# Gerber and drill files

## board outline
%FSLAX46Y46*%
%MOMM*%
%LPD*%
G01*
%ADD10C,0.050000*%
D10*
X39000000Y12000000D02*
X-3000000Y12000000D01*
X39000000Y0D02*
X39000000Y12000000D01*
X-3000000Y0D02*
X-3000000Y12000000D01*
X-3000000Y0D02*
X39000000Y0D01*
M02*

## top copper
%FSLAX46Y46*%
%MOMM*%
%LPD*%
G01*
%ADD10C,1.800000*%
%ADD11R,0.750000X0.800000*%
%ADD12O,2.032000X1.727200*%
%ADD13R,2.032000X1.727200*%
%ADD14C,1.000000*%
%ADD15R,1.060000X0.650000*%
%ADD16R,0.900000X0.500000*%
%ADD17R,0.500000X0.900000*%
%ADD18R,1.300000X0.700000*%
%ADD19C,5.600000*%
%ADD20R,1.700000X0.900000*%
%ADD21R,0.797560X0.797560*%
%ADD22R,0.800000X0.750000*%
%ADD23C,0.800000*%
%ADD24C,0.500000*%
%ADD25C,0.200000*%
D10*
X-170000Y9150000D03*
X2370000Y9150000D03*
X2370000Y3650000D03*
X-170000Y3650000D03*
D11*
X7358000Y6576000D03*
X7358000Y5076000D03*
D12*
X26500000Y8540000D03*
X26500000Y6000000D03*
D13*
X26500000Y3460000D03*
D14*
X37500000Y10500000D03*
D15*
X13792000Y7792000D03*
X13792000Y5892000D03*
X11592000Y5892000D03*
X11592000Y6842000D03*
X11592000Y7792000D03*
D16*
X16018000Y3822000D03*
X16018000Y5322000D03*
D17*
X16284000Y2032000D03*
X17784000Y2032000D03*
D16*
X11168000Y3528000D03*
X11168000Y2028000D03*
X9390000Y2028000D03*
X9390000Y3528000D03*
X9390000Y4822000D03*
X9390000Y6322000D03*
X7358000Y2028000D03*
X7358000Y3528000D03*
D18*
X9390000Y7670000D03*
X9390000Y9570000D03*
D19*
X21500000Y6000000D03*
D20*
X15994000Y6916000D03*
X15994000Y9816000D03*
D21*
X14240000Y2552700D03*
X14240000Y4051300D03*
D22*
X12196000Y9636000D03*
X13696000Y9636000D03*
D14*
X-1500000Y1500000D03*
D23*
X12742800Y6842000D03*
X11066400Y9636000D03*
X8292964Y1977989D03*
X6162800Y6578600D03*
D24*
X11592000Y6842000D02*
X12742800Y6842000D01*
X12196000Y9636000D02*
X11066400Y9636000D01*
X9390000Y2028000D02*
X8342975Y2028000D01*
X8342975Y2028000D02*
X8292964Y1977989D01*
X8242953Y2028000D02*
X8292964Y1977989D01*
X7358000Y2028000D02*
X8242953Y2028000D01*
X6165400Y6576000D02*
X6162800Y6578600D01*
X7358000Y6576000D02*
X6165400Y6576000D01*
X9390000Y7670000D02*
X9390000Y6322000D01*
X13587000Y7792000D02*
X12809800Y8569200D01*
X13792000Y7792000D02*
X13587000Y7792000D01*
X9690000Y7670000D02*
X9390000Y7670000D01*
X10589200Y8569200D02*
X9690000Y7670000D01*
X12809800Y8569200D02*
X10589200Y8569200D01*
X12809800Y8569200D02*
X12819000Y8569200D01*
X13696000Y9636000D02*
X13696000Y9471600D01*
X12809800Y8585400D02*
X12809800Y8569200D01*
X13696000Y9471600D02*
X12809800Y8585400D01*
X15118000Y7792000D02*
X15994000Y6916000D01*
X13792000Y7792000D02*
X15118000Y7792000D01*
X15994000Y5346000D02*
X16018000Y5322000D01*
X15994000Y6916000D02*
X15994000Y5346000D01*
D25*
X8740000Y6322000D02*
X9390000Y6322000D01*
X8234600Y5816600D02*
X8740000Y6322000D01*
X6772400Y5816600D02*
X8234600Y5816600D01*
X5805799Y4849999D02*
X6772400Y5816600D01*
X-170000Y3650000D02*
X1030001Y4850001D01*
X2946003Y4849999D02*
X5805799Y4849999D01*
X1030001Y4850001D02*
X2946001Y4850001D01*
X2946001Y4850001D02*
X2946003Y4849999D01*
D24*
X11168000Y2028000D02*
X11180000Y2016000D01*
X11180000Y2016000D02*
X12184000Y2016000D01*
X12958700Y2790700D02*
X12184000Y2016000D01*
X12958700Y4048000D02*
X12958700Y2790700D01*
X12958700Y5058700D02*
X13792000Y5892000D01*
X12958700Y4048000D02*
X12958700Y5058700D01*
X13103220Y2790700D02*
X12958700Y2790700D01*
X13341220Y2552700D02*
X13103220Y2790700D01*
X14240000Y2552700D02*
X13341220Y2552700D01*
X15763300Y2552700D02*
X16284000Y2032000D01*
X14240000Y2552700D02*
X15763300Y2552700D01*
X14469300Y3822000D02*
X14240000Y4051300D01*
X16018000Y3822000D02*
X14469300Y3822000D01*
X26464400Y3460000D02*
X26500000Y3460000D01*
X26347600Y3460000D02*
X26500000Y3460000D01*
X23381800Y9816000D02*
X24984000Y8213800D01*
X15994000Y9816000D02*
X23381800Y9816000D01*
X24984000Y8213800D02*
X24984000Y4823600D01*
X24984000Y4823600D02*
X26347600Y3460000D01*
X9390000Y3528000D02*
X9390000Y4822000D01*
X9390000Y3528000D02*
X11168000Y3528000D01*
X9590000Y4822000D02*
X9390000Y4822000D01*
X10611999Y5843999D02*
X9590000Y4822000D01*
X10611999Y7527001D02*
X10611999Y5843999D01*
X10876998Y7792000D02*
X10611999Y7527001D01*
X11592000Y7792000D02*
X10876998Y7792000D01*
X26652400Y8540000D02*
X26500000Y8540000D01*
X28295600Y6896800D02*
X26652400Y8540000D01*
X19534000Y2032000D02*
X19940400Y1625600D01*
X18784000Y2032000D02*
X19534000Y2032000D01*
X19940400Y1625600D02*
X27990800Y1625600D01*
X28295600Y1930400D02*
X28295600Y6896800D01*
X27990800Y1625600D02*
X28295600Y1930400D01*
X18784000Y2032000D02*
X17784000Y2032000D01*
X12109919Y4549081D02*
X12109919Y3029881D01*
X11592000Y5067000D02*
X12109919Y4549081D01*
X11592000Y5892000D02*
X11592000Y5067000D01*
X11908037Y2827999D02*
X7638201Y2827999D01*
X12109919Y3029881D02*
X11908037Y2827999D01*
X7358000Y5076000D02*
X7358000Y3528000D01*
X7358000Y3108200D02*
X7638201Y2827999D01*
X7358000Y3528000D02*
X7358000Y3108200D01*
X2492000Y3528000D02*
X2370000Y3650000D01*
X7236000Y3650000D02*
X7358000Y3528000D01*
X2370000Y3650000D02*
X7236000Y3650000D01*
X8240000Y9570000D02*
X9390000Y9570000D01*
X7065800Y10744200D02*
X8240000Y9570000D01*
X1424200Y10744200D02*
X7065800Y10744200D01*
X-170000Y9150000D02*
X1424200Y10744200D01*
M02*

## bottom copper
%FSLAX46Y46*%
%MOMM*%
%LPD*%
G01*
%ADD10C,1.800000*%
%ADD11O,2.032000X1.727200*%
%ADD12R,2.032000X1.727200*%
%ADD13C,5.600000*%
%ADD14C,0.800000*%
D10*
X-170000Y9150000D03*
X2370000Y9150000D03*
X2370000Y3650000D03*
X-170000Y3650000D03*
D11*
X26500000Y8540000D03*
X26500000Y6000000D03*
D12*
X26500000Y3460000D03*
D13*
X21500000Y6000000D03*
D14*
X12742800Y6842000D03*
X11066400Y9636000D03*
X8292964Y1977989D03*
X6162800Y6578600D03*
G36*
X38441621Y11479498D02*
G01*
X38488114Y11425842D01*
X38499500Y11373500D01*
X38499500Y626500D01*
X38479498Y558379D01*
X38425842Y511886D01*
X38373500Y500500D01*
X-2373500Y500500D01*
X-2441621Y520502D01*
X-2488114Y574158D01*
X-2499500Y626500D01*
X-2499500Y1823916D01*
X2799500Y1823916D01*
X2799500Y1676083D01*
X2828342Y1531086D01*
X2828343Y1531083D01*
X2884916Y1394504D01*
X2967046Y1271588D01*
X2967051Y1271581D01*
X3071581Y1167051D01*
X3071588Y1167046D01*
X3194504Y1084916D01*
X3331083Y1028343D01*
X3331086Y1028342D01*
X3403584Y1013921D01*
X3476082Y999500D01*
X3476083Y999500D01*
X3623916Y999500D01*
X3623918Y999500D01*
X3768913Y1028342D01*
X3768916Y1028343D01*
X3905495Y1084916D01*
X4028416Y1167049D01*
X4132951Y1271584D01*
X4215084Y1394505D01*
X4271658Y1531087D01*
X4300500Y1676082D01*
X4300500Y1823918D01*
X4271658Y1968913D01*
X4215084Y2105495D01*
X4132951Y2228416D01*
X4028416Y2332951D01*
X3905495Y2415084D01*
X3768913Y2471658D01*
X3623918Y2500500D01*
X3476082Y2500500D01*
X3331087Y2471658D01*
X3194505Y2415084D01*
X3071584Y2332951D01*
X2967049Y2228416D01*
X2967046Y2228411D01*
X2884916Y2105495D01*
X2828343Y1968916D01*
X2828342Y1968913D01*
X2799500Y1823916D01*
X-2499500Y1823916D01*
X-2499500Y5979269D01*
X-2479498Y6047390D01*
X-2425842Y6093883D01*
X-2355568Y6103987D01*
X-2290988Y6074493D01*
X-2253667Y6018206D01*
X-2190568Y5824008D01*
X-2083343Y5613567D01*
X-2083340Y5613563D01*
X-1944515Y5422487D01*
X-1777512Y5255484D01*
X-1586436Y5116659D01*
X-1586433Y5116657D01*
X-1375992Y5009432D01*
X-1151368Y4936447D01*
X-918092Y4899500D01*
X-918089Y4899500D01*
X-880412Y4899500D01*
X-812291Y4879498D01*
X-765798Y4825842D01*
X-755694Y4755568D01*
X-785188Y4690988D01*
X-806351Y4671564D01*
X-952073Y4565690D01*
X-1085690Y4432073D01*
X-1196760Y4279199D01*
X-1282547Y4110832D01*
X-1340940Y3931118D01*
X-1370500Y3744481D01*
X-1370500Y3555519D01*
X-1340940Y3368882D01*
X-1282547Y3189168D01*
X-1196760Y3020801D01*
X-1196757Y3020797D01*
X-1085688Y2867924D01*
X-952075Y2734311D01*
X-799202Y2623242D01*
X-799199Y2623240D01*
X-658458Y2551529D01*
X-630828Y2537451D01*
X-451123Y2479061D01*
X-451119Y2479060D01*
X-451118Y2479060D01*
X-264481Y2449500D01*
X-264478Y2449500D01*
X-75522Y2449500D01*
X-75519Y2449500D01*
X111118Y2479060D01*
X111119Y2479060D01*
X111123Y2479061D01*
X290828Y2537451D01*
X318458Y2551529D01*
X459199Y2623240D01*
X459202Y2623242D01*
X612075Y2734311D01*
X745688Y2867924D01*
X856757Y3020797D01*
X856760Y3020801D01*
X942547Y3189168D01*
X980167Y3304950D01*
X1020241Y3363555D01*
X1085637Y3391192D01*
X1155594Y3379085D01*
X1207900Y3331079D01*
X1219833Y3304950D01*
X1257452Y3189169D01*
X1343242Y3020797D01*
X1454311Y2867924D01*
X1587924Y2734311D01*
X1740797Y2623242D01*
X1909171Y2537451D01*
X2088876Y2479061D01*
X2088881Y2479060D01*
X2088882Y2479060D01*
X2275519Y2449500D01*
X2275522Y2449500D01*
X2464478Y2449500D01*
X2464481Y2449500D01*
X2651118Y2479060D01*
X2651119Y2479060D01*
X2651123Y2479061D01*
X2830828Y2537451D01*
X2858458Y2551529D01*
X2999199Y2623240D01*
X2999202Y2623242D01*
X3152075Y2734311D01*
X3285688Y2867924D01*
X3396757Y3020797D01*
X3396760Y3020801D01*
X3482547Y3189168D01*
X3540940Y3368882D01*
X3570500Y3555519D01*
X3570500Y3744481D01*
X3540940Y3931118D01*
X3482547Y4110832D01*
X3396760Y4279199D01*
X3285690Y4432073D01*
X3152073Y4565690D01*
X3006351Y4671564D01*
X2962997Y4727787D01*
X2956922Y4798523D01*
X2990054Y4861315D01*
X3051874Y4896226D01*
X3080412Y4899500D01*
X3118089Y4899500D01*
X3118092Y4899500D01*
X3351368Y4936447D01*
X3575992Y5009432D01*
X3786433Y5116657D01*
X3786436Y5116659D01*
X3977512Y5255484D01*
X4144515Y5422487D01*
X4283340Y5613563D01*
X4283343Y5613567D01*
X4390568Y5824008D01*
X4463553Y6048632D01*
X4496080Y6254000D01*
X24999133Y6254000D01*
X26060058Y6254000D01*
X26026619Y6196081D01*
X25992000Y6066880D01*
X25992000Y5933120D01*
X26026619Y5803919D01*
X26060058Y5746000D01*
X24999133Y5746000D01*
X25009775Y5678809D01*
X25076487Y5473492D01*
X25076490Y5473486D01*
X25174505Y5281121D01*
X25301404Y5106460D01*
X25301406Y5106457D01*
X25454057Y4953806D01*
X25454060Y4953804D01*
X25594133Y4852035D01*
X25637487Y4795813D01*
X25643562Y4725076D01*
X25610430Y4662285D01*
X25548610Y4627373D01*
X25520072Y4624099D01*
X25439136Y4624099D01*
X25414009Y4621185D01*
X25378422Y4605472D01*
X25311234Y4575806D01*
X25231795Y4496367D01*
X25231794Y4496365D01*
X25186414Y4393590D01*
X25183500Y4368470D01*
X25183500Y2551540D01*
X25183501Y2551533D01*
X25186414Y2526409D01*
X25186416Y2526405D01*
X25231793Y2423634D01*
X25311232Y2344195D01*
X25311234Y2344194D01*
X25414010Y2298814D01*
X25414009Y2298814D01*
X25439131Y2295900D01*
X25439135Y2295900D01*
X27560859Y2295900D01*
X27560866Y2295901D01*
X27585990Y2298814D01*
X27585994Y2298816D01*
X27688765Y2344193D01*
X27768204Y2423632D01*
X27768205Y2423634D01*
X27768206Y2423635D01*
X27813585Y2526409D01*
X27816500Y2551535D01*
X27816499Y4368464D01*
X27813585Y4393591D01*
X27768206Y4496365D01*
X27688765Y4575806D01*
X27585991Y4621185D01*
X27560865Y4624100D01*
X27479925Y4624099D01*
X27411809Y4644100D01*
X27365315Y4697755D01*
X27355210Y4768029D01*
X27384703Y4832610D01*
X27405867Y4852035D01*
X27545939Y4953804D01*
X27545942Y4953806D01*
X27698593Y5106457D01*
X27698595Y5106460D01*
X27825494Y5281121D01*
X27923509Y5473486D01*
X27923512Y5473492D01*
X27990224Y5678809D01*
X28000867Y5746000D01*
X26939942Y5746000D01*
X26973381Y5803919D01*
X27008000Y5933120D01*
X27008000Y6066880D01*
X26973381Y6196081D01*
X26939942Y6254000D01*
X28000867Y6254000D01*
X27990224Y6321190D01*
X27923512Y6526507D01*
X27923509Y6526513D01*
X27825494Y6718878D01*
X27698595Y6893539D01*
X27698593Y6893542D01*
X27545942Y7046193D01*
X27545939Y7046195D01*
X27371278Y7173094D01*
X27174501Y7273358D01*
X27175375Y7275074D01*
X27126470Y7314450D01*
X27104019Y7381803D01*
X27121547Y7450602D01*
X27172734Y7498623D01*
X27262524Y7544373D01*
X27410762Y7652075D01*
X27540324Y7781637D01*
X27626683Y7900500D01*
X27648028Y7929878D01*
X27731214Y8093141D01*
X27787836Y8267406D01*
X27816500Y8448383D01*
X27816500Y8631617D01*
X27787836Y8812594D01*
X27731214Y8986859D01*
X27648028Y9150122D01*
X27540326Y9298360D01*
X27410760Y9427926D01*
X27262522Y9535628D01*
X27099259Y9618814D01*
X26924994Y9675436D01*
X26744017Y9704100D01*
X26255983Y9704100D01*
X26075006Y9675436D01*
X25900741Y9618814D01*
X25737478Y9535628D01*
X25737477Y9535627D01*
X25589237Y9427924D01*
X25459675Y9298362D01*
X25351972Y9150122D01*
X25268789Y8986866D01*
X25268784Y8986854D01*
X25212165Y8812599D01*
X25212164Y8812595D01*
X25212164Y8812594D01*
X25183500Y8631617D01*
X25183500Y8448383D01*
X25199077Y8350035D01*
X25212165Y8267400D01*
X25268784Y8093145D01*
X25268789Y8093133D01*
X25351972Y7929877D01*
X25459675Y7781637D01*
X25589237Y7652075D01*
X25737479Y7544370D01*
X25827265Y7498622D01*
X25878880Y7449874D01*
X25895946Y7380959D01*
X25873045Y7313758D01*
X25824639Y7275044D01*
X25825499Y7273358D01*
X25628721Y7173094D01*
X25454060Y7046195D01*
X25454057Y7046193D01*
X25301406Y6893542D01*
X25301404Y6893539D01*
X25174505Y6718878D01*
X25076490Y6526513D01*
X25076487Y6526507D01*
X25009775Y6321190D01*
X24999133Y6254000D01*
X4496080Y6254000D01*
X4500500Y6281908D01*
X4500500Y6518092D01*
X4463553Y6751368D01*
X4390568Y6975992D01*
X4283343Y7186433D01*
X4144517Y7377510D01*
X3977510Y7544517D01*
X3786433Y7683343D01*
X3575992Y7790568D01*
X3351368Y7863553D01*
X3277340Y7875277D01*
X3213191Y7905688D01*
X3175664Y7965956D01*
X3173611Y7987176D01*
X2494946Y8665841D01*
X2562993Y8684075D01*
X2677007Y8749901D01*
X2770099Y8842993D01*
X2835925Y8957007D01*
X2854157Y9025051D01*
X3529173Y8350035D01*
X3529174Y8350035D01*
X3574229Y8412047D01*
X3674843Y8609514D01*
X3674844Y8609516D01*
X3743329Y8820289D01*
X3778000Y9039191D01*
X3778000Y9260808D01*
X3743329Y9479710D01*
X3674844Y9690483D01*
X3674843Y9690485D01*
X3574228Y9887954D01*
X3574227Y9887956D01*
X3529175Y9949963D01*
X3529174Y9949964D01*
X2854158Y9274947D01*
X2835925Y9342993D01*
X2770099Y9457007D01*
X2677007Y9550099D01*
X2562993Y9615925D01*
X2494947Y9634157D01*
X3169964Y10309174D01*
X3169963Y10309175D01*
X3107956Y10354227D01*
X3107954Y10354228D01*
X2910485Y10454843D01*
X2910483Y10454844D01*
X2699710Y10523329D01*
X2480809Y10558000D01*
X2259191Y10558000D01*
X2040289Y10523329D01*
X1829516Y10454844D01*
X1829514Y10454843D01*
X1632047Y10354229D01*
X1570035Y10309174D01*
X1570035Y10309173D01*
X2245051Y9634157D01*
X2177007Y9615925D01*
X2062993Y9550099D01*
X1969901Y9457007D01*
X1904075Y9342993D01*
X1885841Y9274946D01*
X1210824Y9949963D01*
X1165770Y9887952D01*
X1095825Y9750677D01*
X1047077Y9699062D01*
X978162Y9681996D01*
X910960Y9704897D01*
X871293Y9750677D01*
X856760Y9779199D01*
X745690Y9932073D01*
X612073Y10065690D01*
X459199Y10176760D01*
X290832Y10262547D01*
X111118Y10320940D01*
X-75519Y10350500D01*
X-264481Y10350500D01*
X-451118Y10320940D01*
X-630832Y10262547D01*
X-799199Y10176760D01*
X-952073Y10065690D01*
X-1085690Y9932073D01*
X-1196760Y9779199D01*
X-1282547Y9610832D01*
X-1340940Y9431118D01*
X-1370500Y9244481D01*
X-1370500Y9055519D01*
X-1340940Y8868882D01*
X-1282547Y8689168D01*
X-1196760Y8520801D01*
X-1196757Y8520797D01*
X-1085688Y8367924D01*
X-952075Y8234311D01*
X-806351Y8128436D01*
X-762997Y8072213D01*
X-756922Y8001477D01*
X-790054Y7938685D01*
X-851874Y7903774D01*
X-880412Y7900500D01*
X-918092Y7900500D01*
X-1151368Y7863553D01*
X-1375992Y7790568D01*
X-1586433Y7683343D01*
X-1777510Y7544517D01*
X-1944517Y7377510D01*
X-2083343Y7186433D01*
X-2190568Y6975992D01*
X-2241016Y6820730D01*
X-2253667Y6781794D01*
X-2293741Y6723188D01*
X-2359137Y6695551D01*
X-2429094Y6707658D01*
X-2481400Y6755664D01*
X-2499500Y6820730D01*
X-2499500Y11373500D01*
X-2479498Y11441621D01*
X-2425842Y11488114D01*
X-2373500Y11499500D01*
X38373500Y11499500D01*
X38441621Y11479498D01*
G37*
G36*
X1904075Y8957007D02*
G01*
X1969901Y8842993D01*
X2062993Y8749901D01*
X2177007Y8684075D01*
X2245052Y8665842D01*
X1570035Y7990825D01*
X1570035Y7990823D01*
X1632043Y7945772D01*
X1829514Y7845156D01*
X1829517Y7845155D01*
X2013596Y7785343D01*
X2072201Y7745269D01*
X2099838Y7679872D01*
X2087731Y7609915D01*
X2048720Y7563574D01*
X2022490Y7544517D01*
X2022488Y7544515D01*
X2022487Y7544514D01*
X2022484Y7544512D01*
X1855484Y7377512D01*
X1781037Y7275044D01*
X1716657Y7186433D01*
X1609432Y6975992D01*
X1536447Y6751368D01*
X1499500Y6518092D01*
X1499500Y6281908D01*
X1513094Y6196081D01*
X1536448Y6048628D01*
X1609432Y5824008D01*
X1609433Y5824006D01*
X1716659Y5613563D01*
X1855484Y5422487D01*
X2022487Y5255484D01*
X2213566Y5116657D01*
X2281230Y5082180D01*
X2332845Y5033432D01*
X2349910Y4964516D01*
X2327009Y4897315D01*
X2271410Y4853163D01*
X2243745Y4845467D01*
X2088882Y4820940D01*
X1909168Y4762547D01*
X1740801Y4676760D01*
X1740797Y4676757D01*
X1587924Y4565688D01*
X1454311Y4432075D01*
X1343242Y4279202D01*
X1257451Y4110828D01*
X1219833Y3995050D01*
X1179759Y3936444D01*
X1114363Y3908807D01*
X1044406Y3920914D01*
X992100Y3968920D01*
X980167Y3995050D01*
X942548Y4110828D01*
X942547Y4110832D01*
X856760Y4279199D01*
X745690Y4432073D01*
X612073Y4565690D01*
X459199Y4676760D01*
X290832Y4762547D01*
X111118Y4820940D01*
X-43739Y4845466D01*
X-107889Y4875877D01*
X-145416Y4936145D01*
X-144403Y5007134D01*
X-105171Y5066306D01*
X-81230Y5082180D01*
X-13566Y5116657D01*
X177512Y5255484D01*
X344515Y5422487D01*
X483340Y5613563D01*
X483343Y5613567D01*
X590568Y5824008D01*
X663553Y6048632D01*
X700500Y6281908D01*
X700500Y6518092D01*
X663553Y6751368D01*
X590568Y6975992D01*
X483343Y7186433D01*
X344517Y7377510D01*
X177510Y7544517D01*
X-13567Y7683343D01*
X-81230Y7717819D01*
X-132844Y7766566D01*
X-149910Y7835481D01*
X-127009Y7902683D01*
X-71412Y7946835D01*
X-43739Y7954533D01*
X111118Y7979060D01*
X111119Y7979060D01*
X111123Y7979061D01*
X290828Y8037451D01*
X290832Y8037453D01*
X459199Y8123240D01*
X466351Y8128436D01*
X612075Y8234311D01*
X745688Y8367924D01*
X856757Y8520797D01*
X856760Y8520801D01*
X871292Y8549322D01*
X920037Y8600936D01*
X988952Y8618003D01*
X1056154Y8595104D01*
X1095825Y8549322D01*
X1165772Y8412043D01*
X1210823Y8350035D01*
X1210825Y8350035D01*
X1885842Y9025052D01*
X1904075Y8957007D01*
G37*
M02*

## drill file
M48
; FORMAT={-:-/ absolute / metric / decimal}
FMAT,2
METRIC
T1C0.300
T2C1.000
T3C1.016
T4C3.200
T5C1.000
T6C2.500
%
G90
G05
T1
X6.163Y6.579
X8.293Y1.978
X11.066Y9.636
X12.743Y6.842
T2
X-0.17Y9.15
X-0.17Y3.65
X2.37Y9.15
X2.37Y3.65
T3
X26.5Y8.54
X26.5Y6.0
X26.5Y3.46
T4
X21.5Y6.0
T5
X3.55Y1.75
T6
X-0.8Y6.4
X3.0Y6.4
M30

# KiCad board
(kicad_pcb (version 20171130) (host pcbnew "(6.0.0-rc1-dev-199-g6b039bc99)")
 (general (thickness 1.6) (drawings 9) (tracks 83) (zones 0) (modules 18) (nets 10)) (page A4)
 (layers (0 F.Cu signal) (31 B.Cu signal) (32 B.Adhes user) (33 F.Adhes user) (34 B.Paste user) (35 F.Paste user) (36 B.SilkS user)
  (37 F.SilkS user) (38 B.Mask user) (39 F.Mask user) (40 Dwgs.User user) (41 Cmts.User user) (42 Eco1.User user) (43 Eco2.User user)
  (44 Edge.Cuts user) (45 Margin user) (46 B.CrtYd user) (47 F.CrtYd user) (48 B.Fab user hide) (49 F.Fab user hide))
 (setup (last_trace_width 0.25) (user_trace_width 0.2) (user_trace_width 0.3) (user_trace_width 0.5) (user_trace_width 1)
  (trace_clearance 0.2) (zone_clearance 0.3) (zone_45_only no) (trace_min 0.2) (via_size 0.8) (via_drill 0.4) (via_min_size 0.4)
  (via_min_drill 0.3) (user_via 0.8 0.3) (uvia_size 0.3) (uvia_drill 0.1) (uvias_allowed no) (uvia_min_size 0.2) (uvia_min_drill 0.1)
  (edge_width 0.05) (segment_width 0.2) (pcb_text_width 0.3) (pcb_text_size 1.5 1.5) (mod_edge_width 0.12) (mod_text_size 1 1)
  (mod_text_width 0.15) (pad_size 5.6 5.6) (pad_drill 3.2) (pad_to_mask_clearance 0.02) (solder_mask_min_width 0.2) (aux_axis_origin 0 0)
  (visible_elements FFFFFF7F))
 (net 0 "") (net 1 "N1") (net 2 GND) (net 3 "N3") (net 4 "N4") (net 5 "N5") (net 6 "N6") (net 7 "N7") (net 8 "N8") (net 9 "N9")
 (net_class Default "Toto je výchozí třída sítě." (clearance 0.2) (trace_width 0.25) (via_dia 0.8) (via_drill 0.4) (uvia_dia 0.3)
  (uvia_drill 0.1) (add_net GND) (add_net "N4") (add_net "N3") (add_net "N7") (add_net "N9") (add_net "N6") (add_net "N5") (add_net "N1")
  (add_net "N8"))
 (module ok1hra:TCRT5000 (layer F.Cu) (at 1.1 -6.4 90)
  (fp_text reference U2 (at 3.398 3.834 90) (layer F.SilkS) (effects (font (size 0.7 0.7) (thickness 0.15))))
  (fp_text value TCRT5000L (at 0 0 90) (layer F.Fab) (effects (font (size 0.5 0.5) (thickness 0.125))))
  (pad "" np_thru_hole circle (at -4.65 2.45 90) (size 1 1) (drill 1) (layers *.Cu *.Mask))
  (pad "" np_thru_hole circle (at 0 1.9 90) (size 2.5 2.5) (drill 2.5) (layers *.Cu *.Mask))
  (pad "" np_thru_hole circle (at 0 -1.9 90) (size 2.5 2.5) (drill 2.5) (layers *.Cu *.Mask))
  (pad 4 thru_hole circle (at 2.75 -1.27 90) (size 1.8 1.8) (drill 1) (layers *.Cu *.Mask) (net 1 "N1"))
  (pad 3 thru_hole circle (at 2.75 1.27 90) (size 1.8 1.8) (drill 1) (layers *.Cu *.Mask) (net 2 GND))
  (pad 2 thru_hole circle (at -2.75 1.27 90) (size 1.8 1.8) (drill 1) (layers *.Cu *.Mask) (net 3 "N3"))
  (pad 1 thru_hole circle (at -2.75 -1.27 90) (size 1.8 1.8) (drill 1) (layers *.Cu *.Mask) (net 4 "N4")))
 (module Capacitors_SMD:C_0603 (layer F.Cu) (at 7.358 -5.826 90)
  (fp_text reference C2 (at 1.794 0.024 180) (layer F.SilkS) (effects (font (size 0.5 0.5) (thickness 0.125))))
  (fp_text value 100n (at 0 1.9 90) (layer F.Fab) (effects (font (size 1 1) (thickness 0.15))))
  (pad 2 smd rect (at 0.75 0 90) (size 0.8 0.75) (layers F.Cu F.Paste F.Mask) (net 2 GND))
  (pad 1 smd rect (at -0.75 0 90) (size 0.8 0.75) (layers F.Cu F.Paste F.Mask) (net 3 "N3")))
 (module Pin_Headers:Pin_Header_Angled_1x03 (layer B.Cu) (at 26.5 -3.46)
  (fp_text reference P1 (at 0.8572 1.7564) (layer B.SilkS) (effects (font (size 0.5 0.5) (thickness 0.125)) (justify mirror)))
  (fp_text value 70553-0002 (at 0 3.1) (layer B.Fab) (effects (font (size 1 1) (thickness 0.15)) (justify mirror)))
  (pad 3 thru_hole oval (at 0 -5.08) (size 2.032 1.7272) (drill 1.016) (layers *.Cu *.Mask) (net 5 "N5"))
  (pad 2 thru_hole oval (at 0 -2.54) (size 2.032 1.7272) (drill 1.016) (layers *.Cu *.Mask) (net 2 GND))
  (pad 1 thru_hole rect (at 0 0) (size 2.032 1.7272) (drill 1.016) (layers *.Cu *.Mask) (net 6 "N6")))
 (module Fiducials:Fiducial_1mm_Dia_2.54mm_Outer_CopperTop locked (layer F.Cu) (at 37.5 -10.5)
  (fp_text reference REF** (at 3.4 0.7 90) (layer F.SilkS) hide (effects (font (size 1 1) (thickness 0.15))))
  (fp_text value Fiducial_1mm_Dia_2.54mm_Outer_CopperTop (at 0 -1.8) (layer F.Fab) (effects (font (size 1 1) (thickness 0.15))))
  (pad ~ smd circle (at 0 0) (size 1 1) (layers F.Cu F.Mask) (solder_mask_margin 0.77) (clearance 0.77)))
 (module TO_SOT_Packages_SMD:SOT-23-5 (layer F.Cu) (at 12.692 -6.842)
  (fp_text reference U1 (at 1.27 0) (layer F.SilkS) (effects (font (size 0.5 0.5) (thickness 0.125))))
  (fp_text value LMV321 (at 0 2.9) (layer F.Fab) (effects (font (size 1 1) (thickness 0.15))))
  (pad 5 smd rect (at 1.1 -0.95) (size 1.06 0.65) (layers F.Cu F.Paste F.Mask) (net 4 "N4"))
  (pad 4 smd rect (at 1.1 0.95) (size 1.06 0.65) (layers F.Cu F.Paste F.Mask) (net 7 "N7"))
  (pad 3 smd rect (at -1.1 0.95) (size 1.06 0.65) (layers F.Cu F.Paste F.Mask) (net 3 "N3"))
  (pad 2 smd rect (at -1.1 0) (size 1.06 0.65) (layers F.Cu F.Paste F.Mask) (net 2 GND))
  (pad 1 smd rect (at -1.1 -0.95) (size 1.06 0.65) (layers F.Cu F.Paste F.Mask) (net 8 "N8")))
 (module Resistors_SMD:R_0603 (layer F.Cu) (at 16.018 -4.572 270)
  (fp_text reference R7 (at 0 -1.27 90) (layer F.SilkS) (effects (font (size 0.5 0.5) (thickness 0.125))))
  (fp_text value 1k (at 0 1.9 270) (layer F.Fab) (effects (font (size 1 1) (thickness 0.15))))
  (pad 2 smd rect (at 0.75 0 270) (size 0.5 0.9) (layers F.Cu F.Paste F.Mask) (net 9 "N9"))
  (pad 1 smd rect (at -0.75 0 270) (size 0.5 0.9) (layers F.Cu F.Paste F.Mask) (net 4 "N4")))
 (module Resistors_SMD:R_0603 (layer F.Cu) (at 17.034 -2.032 180)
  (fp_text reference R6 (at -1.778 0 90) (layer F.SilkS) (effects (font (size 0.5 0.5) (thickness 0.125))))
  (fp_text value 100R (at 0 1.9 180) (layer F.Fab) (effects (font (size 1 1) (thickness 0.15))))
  (pad 2 smd rect (at 0.75 0 180) (size 0.5 0.9) (layers F.Cu F.Paste F.Mask) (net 7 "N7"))
  (pad 1 smd rect (at -0.75 0 180) (size 0.5 0.9) (layers F.Cu F.Paste F.Mask) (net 5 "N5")))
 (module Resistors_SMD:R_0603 (layer F.Cu) (at 11.168 -2.778 90)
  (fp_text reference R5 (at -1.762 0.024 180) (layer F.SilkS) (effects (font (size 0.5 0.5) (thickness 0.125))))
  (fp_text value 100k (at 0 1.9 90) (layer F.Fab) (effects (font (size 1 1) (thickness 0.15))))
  (pad 2 smd rect (at 0.75 0 90) (size 0.5 0.9) (layers F.Cu F.Paste F.Mask) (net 8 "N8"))
  (pad 1 smd rect (at -0.75 0 90) (size 0.5 0.9) (layers F.Cu F.Paste F.Mask) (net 7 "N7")))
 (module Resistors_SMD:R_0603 (layer F.Cu) (at 9.39 -2.778 270)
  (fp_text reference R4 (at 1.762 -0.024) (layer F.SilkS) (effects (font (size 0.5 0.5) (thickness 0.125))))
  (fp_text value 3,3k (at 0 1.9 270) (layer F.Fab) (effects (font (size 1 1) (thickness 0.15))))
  (pad 2 smd rect (at 0.75 0 270) (size 0.5 0.9) (layers F.Cu F.Paste F.Mask) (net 2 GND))
  (pad 1 smd rect (at -0.75 0 270) (size 0.5 0.9) (layers F.Cu F.Paste F.Mask) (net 8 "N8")))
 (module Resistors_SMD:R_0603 (layer F.Cu) (at 9.39 -5.572 270)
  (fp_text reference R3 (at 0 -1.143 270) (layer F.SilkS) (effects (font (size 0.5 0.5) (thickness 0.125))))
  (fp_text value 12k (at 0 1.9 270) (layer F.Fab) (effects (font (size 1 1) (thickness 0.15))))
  (pad 2 smd rect (at 0.75 0 270) (size 0.5 0.9) (layers F.Cu F.Paste F.Mask) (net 8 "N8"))
  (pad 1 smd rect (at -0.75 0 270) (size 0.5 0.9) (layers F.Cu F.Paste F.Mask) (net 4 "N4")))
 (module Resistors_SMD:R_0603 (layer F.Cu) (at 7.358 -2.778 270)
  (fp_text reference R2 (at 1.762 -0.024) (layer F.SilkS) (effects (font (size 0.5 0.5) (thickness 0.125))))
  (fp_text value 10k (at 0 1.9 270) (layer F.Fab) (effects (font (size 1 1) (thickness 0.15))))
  (pad 2 smd rect (at 0.75 0 270) (size 0.5 0.9) (layers F.Cu F.Paste F.Mask) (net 2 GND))
  (pad 1 smd rect (at -0.75 0 270) (size 0.5 0.9) (layers F.Cu F.Paste F.Mask) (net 3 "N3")))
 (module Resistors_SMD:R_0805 (layer F.Cu) (at 9.39 -8.62 270)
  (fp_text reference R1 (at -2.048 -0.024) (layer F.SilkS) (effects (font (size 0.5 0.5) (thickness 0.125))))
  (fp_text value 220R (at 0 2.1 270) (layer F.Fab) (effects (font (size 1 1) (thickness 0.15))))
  (pad 2 smd rect (at 0.95 0 270) (size 0.7 1.3) (layers F.Cu F.Paste F.Mask) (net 4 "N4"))
  (pad 1 smd rect (at -0.95 0 270) (size 0.7 1.3) (layers F.Cu F.Paste F.Mask) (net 1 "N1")))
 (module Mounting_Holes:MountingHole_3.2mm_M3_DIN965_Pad (layer F.Cu) (at 21.5 -6)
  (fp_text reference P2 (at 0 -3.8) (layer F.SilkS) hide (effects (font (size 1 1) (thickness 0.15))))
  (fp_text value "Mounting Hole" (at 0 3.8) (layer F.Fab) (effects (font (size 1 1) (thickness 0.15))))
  (pad 1 thru_hole circle (at 0 0) (size 5.6 5.6) (drill 3.2) (layers *.Cu *.Mask) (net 2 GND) (zone_connect 2)))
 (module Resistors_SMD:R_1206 (layer F.Cu) (at 15.994 -8.366 270)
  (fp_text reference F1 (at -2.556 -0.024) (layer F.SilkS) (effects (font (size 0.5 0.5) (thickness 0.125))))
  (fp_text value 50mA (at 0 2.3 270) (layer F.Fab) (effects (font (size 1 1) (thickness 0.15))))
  (pad 2 smd rect (at 1.45 0 270) (size 0.9 1.7) (layers F.Cu F.Paste F.Mask) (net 4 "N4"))
  (pad 1 smd rect (at -1.45 0 270) (size 0.9 1.7) (layers F.Cu F.Paste F.Mask) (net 6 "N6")))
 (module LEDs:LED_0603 (layer F.Cu) (at 14.24 -3.302 90)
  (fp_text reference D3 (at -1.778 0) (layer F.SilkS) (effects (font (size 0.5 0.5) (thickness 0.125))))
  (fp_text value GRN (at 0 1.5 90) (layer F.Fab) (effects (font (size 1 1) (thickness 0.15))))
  (pad 1 smd rect (at -0.7493 0 270) (size 0.79756 0.79756) (layers F.Cu F.Paste F.Mask) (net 7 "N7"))
  (pad 2 smd rect (at 0.7493 0 270) (size 0.79756 0.79756) (layers F.Cu F.Paste F.Mask) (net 9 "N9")))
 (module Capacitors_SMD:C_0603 (layer F.Cu) (at 12.946 -9.636 180)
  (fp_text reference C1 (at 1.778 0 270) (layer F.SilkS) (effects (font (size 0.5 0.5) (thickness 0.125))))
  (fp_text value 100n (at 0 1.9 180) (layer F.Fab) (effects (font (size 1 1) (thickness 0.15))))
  (pad 2 smd rect (at 0.75 0 180) (size 0.8 0.75) (layers F.Cu F.Paste F.Mask) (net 2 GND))
  (pad 1 smd rect (at -0.75 0 180) (size 0.8 0.75) (layers F.Cu F.Paste F.Mask) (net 4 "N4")))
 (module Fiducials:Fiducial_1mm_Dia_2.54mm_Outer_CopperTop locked (layer F.Cu) (at -1.5 -1.5)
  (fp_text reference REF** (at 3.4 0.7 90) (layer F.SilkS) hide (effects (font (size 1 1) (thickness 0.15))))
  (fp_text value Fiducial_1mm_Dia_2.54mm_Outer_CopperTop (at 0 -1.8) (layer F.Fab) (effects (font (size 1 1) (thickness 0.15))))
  (pad ~ smd circle (at 0 0) (size 1 1) (layers F.Cu F.Mask) (solder_mask_margin 0.77) (clearance 0.77)))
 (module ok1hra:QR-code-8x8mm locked (layer B.Cu) (at 11 -6 180)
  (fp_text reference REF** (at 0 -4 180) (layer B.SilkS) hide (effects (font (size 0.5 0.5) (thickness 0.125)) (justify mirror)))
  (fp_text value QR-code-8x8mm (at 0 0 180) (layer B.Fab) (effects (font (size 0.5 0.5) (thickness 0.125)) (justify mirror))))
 (gr_line (start 39 -12) (end -3 -12) (layer Edge.Cuts) (width 0.05))
 (gr_line (start 39 0) (end 39 -12) (layer Edge.Cuts) (width 0.05))
 (gr_line (start -3 0) (end -3 -12) (layer Edge.Cuts) (width 0.05))
 (gr_line (start -3 0) (end 39 0) (layer Edge.Cuts) (width 0.05))
 (via (at 12.7428 -6.842) (size 0.8) (drill 0.3) (layers F.Cu B.Cu) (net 2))
 (segment (start 11.592 -6.842) (end 12.7428 -6.842) (width 0.5) (layer F.Cu) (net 2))
 (via (at 11.0664 -9.636) (size 0.8) (drill 0.3) (layers F.Cu B.Cu) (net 2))
 (segment (start 12.196 -9.636) (end 11.0664 -9.636) (width 0.5) (layer F.Cu) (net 2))
 (segment (start 9.39 -2.028) (end 8.342975 -2.028) (width 0.5) (layer F.Cu) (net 2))
 (segment (start 8.342975 -2.028) (end 8.292964 -1.977989) (width 0.5) (layer F.Cu) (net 2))
 (via (at 8.292964 -1.977989) (size 0.8) (drill 0.3) (layers F.Cu B.Cu) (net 2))
 (segment (start 8.242953 -2.028) (end 8.292964 -1.977989) (width 0.5) (layer F.Cu) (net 2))
 (segment (start 7.358 -2.028) (end 8.242953 -2.028) (width 0.5) (layer F.Cu) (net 2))
 (segment (start 6.1654 -6.576) (end 6.1628 -6.5786) (width 0.5) (layer F.Cu) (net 2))
 (via (at 6.1628 -6.5786) (size 0.8) (drill 0.3) (layers F.Cu B.Cu) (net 2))
 (segment (start 7.358 -6.576) (end 6.1654 -6.576) (width 0.5) (layer F.Cu) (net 2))
 (segment (start 9.39 -7.67) (end 9.39 -6.322) (width 0.5) (layer F.Cu) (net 4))
 (segment (start 13.587 -7.792) (end 12.8098 -8.5692) (width 0.5) (layer F.Cu) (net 4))
 (segment (start 13.792 -7.792) (end 13.587 -7.792) (width 0.5) (layer F.Cu) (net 4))
 (segment (start 9.69 -7.67) (end 9.39 -7.67) (width 0.5) (layer F.Cu) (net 4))
 (segment (start 10.5892 -8.5692) (end 9.69 -7.67) (width 0.5) (layer F.Cu) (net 4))
 (segment (start 12.8098 -8.5692) (end 10.5892 -8.5692) (width 0.5) (layer F.Cu) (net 4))
 (segment (start 12.8098 -8.5692) (end 12.819 -8.5692) (width 0.5) (layer F.Cu) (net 4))
 (segment (start 13.696 -9.636) (end 13.696 -9.4716) (width 0.5) (layer F.Cu) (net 4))
 (segment (start 12.8098 -8.5854) (end 12.8098 -8.5692) (width 0.5) (layer F.Cu) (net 4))
 (segment (start 13.696 -9.4716) (end 12.8098 -8.5854) (width 0.5) (layer F.Cu) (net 4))
 (segment (start 15.118 -7.792) (end 15.994 -6.916) (width 0.5) (layer F.Cu) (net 4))
 (segment (start 13.792 -7.792) (end 15.118 -7.792) (width 0.5) (layer F.Cu) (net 4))
 (segment (start 15.994 -5.346) (end 16.018 -5.322) (width 0.5) (layer F.Cu) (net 4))
 (segment (start 15.994 -6.916) (end 15.994 -5.346) (width 0.5) (layer F.Cu) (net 4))
 (segment (start 8.74 -6.322) (end 9.39 -6.322) (width 0.2) (layer F.Cu) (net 4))
 (segment (start 8.2346 -5.8166) (end 8.74 -6.322) (width 0.2) (layer F.Cu) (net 4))
 (segment (start 6.7724 -5.8166) (end 8.2346 -5.8166) (width 0.2) (layer F.Cu) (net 4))
 (segment (start 5.805799 -4.849999) (end 6.7724 -5.8166) (width 0.2) (layer F.Cu) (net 4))
 (segment (start -0.17 -3.65) (end 1.030001 -4.850001) (width 0.2) (layer F.Cu) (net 4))
 (segment (start 2.946003 -4.849999) (end 5.805799 -4.849999) (width 0.2) (layer F.Cu) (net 4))
 (segment (start 1.030001 -4.850001) (end 2.946001 -4.850001) (width 0.2) (layer F.Cu) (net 4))
 (segment (start 2.946001 -4.850001) (end 2.946003 -4.849999) (width 0.2) (layer F.Cu) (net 4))
 (segment (start 11.168 -2.028) (end 11.18 -2.016) (width 0.5) (layer F.Cu) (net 7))
 (segment (start 11.18 -2.016) (end 12.184 -2.016) (width 0.5) (layer F.Cu) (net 7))
 (segment (start 12.9587 -2.7907) (end 12.184 -2.016) (width 0.5) (layer F.Cu) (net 7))
 (segment (start 12.9587 -4.048) (end 12.9587 -2.7907) (width 0.5) (layer F.Cu) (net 7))
 (segment (start 12.9587 -5.0587) (end 13.792 -5.892) (width 0.5) (layer F.Cu) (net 7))
 (segment (start 12.9587 -4.048) (end 12.9587 -5.0587) (width 0.5) (layer F.Cu) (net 7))
 (segment (start 13.10322 -2.7907) (end 12.9587 -2.7907) (width 0.5) (layer F.Cu) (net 7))
 (segment (start 13.34122 -2.5527) (end 13.10322 -2.7907) (width 0.5) (layer F.Cu) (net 7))
 (segment (start 14.24 -2.5527) (end 13.34122 -2.5527) (width 0.5) (layer F.Cu) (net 7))
 (segment (start 15.7633 -2.5527) (end 16.284 -2.032) (width 0.5) (layer F.Cu) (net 7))
 (segment (start 14.24 -2.5527) (end 15.7633 -2.5527) (width 0.5) (layer F.Cu) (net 7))
 (segment (start 14.4693 -3.822) (end 14.24 -4.0513) (width 0.5) (layer F.Cu) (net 9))
 (segment (start 16.018 -3.822) (end 14.4693 -3.822) (width 0.5) (layer F.Cu) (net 9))
 (segment (start 26.4644 -3.46) (end 26.5 -3.46) (width 0.5) (layer F.Cu) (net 6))
 (segment (start 26.3476 -3.46) (end 26.5 -3.46) (width 0.5) (layer F.Cu) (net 6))
 (segment (start 23.3818 -9.816) (end 24.984 -8.2138) (width 0.5) (layer F.Cu) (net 6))
 (segment (start 15.994 -9.816) (end 23.3818 -9.816) (width 0.5) (layer F.Cu) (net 6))
 (segment (start 24.984 -8.2138) (end 24.984 -4.8236) (width 0.5) (layer F.Cu) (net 6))
 (segment (start 24.984 -4.8236) (end 26.3476 -3.46) (width 0.5) (layer F.Cu) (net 6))
 (segment (start 9.39 -3.528) (end 9.39 -4.822) (width 0.5) (layer F.Cu) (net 8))
 (segment (start 9.39 -3.528) (end 11.168 -3.528) (width 0.5) (layer F.Cu) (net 8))
 (segment (start 9.59 -4.822) (end 9.39 -4.822) (width 0.5) (layer F.Cu) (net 8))
 (segment (start 10.611999 -5.843999) (end 9.59 -4.822) (width 0.5) (layer F.Cu) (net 8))
 (segment (start 10.611999 -7.527001) (end 10.611999 -5.843999) (width 0.5) (layer F.Cu) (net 8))
 (segment (start 10.876998 -7.792) (end 10.611999 -7.527001) (width 0.5) (layer F.Cu) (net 8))
 (segment (start 11.592 -7.792) (end 10.876998 -7.792) (width 0.5) (layer F.Cu) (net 8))
 (segment (start 26.6524 -8.54) (end 26.5 -8.54) (width 0.5) (layer F.Cu) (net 5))
 (segment (start 28.2956 -6.8968) (end 26.6524 -8.54) (width 0.5) (layer F.Cu) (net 5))
 (segment (start 19.534 -2.032) (end 19.9404 -1.6256) (width 0.5) (layer F.Cu) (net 5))
 (segment (start 18.784 -2.032) (end 19.534 -2.032) (width 0.5) (layer F.Cu) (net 5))
 (segment (start 19.9404 -1.6256) (end 27.9908 -1.6256) (width 0.5) (layer F.Cu) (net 5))
 (segment (start 28.2956 -1.9304) (end 28.2956 -6.8968) (width 0.5) (layer F.Cu) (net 5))
 (segment (start 27.9908 -1.6256) (end 28.2956 -1.9304) (width 0.5) (layer F.Cu) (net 5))
 (segment (start 18.784 -2.032) (end 17.784 -2.032) (width 0.5) (layer F.Cu) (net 5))
 (segment (start 12.109919 -4.549081) (end 12.109919 -3.029881) (width 0.5) (layer F.Cu) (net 3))
 (segment (start 11.592 -5.067) (end 12.109919 -4.549081) (width 0.5) (layer F.Cu) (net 3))
 (segment (start 11.592 -5.892) (end 11.592 -5.067) (width 0.5) (layer F.Cu) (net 3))
 (segment (start 11.908037 -2.827999) (end 7.638201 -2.827999) (width 0.5) (layer F.Cu) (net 3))
 (segment (start 12.109919 -3.029881) (end 11.908037 -2.827999) (width 0.5) (layer F.Cu) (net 3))
 (segment (start 7.358 -5.076) (end 7.358 -3.528) (width 0.5) (layer F.Cu) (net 3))
 (segment (start 7.358 -3.1082) (end 7.638201 -2.827999) (width 0.5) (layer F.Cu) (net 3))
 (segment (start 7.358 -3.528) (end 7.358 -3.1082) (width 0.5) (layer F.Cu) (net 3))
 (segment (start 2.492 -3.528) (end 2.37 -3.65) (width 0.5) (layer F.Cu) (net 3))
 (segment (start 7.236 -3.65) (end 7.358 -3.528) (width 0.5) (layer F.Cu) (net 3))
 (segment (start 2.37 -3.65) (end 7.236 -3.65) (width 0.5) (layer F.Cu) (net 3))
 (segment (start 8.24 -9.57) (end 9.39 -9.57) (width 0.5) (layer F.Cu) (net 1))
 (segment (start 7.0658 -10.7442) (end 8.24 -9.57) (width 0.5) (layer F.Cu) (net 1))
 (segment (start 1.4242 -10.7442) (end 7.0658 -10.7442) (width 0.5) (layer F.Cu) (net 1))
 (segment (start -0.17 -9.15) (end 1.4242 -10.7442) (width 0.5) (layer F.Cu) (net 1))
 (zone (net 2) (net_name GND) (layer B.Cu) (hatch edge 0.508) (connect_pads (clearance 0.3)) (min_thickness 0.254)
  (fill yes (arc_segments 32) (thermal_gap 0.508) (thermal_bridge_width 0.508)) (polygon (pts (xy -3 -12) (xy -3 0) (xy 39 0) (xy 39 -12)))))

